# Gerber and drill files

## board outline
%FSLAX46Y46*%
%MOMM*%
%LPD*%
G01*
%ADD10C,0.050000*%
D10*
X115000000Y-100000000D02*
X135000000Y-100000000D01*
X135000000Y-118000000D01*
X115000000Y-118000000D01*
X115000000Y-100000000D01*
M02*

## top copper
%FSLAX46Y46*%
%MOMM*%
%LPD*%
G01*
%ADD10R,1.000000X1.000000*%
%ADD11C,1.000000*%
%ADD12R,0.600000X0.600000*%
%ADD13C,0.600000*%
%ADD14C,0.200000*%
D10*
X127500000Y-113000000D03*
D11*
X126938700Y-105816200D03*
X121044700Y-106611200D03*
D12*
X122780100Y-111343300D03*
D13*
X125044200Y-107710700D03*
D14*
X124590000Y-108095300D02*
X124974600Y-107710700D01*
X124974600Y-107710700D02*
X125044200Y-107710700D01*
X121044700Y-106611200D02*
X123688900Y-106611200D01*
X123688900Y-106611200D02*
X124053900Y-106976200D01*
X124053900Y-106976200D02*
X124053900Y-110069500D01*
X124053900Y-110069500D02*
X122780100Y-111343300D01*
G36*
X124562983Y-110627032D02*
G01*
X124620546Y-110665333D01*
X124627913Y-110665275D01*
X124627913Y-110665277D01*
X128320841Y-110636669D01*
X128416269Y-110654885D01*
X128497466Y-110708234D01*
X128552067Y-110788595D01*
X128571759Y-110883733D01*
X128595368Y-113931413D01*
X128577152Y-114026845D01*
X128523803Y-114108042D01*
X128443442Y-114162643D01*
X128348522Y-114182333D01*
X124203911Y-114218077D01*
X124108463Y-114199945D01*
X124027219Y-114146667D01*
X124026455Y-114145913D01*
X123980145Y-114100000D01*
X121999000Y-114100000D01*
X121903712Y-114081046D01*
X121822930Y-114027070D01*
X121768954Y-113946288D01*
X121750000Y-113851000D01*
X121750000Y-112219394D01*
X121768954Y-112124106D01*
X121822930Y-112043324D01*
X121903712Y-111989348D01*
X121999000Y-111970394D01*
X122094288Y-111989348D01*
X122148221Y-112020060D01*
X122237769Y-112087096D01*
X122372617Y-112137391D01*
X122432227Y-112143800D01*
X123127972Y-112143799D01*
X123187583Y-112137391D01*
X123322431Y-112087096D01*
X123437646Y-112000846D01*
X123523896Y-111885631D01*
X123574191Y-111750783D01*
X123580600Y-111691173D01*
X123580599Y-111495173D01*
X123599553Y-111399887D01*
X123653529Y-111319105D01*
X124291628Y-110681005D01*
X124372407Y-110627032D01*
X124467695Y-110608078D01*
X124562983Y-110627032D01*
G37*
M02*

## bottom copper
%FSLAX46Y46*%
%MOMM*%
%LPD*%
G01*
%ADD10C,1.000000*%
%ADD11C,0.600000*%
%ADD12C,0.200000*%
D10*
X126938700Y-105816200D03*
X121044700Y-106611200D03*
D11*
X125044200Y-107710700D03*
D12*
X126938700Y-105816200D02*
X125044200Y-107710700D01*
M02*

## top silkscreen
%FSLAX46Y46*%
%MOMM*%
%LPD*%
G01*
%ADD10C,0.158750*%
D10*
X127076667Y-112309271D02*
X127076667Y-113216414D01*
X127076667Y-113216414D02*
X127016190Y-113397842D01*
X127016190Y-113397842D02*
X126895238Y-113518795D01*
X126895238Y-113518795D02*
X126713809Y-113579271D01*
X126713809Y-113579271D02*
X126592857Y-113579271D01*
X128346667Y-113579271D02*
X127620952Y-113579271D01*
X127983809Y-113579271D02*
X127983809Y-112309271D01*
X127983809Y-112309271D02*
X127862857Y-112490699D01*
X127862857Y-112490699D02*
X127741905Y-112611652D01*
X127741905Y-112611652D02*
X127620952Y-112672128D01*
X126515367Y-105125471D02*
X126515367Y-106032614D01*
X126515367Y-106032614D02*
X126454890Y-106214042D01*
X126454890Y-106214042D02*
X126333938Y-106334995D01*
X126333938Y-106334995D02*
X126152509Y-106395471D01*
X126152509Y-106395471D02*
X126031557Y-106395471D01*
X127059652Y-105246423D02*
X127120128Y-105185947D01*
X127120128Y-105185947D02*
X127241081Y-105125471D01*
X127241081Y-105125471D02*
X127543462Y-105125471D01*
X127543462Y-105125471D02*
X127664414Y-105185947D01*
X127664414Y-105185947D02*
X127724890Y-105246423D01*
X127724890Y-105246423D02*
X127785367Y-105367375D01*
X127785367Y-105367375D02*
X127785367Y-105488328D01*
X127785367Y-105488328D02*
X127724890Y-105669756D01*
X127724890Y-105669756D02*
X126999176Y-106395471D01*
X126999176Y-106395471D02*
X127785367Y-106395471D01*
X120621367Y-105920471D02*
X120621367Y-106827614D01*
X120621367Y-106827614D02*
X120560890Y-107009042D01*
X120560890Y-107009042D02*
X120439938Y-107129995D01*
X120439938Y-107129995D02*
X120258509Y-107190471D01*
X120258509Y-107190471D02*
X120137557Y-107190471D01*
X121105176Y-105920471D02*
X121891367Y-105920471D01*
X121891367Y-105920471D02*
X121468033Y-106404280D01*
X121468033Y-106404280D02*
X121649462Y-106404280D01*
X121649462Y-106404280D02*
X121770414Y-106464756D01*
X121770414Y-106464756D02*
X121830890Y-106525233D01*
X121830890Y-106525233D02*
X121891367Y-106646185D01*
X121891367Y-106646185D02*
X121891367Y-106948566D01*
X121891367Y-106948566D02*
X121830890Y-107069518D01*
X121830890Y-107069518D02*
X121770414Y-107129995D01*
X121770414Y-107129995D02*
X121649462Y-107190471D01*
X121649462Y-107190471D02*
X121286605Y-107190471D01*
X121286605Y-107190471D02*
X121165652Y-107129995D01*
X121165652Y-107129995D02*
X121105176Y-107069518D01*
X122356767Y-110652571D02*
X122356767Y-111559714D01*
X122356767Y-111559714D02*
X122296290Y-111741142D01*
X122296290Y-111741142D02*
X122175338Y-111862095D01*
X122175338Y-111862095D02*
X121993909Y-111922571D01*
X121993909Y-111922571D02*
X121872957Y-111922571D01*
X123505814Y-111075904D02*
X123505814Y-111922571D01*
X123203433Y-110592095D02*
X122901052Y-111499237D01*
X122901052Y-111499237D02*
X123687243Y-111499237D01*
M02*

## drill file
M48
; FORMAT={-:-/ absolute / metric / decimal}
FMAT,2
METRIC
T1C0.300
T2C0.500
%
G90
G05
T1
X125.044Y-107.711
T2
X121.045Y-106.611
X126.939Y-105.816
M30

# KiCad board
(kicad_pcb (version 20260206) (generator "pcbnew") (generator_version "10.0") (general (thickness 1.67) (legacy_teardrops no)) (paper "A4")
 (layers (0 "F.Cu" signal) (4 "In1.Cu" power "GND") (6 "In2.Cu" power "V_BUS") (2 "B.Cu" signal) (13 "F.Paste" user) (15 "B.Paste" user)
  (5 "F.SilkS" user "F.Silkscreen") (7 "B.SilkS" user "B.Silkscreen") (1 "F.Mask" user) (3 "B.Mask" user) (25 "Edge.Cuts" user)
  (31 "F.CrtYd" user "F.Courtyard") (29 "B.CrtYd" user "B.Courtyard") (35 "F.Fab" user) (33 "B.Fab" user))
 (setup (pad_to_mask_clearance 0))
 (gr_rect (start 115 100) (end 135 118) (stroke (width 0.05) (type default)) (fill no) (layer "Edge.Cuts"))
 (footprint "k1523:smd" (layer "F.Cu") (at 127.5 113.0) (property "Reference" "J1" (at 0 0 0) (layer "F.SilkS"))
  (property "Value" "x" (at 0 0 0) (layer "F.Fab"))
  (pad "1" smd rect (at 0 0) (size 1 1) (layers "F.Cu" "F.Mask") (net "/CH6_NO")))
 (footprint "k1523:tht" (layer "F.Cu") (at 126.9387 105.8162) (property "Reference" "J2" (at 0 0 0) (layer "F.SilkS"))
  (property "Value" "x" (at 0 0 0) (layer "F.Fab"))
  (pad "1" thru_hole circle (at 0 0) (size 1 1) (drill 0.5) (layers "*.Cu" "*.Mask") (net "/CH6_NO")))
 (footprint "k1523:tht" (layer "F.Cu") (at 121.0447 106.6112) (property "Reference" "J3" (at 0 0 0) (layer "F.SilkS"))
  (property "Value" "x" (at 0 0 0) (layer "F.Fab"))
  (pad "1" thru_hole circle (at 0 0) (size 1 1) (drill 0.5) (layers "*.Cu" "*.Mask") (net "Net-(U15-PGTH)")))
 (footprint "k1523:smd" (layer "F.Cu") (at 122.7801 111.3433) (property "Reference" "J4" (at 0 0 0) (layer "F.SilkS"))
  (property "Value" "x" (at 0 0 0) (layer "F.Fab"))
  (pad "1" smd rect (at 0 0) (size 0.6 0.6) (layers "F.Cu" "F.Mask") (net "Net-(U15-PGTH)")))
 (segment (start 124.59 108.0953) (end 124.9746 107.7107) (width 0.2) (layer "F.Cu") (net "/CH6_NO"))
 (segment (start 124.9746 107.7107) (end 125.0442 107.7107) (width 0.2) (layer "F.Cu") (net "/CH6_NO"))
 (via (at 125.0442 107.7107) (size 0.6) (drill 0.3) (layers "F.Cu" "B.Cu") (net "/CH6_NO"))
 (segment (start 126.9387 105.8162) (end 125.0442 107.7107) (width 0.2) (layer "B.Cu") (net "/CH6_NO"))
 (segment (start 121.0447 106.6112) (end 123.6889 106.6112) (width 0.2) (layer "F.Cu") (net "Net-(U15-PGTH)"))
 (segment (start 123.6889 106.6112) (end 124.0539 106.9762) (width 0.2) (layer "F.Cu") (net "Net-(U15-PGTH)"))
 (segment (start 124.0539 106.9762) (end 124.0539 110.0695) (width 0.2) (layer "F.Cu") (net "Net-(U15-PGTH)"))
 (segment (start 124.0539 110.0695) (end 122.7801 111.3433) (width 0.2) (layer "F.Cu") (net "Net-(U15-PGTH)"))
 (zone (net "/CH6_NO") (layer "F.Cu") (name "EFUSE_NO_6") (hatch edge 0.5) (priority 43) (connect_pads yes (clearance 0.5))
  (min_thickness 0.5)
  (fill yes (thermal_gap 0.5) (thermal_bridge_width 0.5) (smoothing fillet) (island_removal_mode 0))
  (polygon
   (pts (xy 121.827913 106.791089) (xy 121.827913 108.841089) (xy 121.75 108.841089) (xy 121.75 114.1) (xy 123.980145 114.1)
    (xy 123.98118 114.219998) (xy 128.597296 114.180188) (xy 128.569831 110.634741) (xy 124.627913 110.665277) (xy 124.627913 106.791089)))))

